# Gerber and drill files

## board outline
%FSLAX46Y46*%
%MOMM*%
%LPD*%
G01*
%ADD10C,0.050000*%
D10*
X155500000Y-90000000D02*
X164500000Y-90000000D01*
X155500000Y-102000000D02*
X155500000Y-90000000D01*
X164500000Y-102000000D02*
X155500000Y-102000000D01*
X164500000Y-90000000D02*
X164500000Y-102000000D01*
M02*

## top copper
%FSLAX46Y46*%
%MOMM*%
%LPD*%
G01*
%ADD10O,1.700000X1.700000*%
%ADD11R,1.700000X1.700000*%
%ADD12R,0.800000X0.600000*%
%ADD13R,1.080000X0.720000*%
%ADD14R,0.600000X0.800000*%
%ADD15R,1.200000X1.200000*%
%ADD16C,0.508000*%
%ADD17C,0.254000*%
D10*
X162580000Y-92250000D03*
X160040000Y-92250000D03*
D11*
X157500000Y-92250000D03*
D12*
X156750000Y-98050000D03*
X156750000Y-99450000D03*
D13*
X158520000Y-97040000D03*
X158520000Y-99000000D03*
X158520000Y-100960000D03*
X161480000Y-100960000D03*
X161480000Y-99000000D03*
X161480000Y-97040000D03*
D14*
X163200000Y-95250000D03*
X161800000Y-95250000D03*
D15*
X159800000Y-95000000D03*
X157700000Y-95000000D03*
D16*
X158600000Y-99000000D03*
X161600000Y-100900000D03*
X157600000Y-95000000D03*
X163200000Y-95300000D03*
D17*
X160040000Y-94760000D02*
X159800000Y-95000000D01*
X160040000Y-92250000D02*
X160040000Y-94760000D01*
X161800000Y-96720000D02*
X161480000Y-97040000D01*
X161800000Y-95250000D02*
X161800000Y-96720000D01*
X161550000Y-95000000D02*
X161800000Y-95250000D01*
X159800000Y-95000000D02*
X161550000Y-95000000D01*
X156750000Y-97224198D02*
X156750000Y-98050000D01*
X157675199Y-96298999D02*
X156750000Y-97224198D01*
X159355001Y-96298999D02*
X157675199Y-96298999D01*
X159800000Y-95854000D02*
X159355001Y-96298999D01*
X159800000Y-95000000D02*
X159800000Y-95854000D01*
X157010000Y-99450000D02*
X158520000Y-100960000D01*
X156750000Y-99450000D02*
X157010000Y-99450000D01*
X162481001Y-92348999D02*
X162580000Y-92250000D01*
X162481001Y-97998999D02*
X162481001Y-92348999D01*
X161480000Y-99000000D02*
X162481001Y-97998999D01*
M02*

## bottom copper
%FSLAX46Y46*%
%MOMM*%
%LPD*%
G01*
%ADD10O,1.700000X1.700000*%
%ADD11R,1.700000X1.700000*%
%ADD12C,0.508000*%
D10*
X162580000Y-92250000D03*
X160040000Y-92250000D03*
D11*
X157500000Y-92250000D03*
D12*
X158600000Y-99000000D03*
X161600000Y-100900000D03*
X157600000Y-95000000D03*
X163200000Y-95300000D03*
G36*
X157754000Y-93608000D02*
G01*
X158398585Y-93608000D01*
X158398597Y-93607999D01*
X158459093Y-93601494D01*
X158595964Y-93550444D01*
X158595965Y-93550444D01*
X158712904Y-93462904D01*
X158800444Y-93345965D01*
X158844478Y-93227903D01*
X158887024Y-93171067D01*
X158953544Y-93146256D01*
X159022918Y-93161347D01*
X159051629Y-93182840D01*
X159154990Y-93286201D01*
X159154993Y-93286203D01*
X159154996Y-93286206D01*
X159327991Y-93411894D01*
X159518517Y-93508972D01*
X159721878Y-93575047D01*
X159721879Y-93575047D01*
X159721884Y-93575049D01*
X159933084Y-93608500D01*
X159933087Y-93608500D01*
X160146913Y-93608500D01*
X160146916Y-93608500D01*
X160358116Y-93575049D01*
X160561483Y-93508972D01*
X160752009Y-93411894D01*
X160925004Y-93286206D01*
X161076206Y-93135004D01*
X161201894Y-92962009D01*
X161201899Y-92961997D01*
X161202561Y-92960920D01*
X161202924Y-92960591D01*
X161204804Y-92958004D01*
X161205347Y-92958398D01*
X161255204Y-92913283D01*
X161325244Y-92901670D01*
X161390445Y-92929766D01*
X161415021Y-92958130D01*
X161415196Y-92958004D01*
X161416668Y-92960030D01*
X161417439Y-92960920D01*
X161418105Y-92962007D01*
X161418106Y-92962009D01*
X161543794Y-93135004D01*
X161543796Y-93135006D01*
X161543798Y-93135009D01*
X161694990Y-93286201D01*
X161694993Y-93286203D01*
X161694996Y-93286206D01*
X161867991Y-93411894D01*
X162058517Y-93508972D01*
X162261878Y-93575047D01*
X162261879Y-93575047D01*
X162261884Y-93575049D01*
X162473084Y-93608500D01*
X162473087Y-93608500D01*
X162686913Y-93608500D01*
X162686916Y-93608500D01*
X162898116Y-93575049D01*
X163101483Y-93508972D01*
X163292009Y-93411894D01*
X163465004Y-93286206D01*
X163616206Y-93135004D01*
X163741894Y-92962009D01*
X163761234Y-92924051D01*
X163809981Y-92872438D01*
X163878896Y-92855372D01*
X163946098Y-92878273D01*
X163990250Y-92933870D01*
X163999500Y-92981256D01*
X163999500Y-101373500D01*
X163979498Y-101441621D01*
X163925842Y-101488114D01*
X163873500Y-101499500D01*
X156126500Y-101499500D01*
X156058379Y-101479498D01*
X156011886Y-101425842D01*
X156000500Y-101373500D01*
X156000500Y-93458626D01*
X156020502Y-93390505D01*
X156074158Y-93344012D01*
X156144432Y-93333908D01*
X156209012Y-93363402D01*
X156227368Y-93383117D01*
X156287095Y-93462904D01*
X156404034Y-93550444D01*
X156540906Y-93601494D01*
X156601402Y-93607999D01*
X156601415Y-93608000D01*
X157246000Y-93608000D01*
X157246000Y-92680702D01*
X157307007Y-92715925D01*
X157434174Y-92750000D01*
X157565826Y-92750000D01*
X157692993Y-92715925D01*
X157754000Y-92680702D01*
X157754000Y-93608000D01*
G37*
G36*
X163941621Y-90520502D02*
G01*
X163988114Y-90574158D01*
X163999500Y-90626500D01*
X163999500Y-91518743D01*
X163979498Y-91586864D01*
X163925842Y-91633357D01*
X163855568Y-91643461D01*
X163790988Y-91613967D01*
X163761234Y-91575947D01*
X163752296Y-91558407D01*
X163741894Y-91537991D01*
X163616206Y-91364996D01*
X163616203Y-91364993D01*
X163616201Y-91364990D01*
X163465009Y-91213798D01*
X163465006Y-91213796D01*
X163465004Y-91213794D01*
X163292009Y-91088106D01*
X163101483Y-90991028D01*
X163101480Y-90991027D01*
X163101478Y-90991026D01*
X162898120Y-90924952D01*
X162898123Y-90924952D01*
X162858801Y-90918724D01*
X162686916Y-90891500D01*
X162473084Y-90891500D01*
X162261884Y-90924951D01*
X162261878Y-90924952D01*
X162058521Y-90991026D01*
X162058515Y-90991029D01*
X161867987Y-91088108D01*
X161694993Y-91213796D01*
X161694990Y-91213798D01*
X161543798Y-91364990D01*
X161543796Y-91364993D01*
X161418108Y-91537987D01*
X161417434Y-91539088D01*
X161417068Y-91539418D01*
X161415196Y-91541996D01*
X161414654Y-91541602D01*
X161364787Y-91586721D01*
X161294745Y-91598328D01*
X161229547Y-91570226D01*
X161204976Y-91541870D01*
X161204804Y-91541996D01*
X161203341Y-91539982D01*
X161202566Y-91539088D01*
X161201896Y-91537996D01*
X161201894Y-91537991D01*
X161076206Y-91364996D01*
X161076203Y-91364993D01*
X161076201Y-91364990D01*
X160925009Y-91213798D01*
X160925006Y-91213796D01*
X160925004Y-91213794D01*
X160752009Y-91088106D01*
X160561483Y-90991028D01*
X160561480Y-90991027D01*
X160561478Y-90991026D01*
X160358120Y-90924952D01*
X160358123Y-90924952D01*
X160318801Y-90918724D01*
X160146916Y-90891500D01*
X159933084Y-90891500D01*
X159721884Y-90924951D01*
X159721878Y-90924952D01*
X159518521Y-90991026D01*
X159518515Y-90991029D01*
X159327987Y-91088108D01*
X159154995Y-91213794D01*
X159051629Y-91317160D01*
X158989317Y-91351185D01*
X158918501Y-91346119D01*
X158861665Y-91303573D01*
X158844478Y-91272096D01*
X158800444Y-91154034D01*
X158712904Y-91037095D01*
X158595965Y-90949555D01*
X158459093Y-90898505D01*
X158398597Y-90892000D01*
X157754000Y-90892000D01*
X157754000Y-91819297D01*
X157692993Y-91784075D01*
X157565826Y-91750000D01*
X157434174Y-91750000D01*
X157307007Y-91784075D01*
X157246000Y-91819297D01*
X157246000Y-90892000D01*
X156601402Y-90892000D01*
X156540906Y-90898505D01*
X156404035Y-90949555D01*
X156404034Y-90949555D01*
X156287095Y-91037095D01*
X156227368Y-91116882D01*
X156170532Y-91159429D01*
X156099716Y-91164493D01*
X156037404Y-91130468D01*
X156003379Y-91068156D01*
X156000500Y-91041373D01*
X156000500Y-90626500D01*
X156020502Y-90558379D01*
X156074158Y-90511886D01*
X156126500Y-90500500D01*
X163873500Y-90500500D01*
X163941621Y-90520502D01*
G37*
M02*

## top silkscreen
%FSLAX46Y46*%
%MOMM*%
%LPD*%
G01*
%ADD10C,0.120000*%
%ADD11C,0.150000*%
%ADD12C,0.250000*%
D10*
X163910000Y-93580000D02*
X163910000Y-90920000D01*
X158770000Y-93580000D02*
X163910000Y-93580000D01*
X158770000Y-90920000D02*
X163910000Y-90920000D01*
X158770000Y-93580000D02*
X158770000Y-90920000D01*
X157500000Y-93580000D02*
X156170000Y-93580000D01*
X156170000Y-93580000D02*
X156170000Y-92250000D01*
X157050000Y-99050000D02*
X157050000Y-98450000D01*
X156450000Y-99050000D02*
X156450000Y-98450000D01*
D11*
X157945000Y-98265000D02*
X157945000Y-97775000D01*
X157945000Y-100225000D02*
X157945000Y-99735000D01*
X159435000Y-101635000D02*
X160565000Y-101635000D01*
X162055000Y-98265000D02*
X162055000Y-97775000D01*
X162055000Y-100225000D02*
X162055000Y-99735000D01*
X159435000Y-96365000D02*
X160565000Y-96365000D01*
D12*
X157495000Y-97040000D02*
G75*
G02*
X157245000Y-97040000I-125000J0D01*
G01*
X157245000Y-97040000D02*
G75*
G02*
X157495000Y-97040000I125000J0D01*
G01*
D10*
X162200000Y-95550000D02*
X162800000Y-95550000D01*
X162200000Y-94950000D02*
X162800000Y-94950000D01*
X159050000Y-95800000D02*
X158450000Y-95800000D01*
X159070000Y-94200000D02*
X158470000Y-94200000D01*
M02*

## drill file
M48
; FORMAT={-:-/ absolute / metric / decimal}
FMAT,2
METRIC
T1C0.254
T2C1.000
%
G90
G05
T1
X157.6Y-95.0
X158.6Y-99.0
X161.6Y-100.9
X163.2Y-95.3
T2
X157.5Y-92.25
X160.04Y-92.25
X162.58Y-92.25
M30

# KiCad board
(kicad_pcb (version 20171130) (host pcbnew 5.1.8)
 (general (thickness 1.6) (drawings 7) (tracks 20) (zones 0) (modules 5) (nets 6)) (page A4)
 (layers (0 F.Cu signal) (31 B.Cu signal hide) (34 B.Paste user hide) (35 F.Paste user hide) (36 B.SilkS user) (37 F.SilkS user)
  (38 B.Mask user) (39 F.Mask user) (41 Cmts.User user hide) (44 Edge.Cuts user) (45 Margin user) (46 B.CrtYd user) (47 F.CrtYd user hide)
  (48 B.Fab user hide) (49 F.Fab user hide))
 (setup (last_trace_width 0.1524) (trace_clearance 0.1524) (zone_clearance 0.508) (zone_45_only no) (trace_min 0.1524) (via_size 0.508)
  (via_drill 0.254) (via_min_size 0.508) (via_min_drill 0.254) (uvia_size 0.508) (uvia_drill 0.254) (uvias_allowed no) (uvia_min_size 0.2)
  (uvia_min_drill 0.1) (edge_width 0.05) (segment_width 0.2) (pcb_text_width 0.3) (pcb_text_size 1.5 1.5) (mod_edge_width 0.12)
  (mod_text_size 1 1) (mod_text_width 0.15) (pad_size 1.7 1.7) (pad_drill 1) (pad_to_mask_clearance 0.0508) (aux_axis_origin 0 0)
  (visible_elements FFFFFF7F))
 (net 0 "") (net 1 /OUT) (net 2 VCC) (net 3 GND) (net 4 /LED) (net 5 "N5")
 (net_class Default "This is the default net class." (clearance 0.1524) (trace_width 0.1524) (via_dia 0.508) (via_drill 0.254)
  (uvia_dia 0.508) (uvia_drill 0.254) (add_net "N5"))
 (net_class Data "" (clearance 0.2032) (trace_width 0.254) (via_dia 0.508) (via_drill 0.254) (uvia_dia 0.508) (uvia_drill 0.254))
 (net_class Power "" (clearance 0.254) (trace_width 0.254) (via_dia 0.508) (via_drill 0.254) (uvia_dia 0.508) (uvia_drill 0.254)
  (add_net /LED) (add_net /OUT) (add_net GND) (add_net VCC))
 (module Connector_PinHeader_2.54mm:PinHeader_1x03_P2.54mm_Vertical (layer F.Cu) (at 157.5 92.25 90)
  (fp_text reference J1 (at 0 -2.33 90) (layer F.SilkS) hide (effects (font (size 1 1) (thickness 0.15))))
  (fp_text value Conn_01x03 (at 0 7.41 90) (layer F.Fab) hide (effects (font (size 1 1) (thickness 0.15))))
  (fp_line (start -1.33 6.41) (end 1.33 6.41) (layer F.SilkS) (width 0.12))
  (fp_line (start -1.33 1.27) (end -1.33 6.41) (layer F.SilkS) (width 0.12))
  (fp_line (start 1.33 1.27) (end 1.33 6.41) (layer F.SilkS) (width 0.12))
  (fp_line (start -1.33 1.27) (end 1.33 1.27) (layer F.SilkS) (width 0.12))
  (fp_line (start -1.33 0) (end -1.33 -1.33) (layer F.SilkS) (width 0.12))
  (fp_line (start -1.33 -1.33) (end 0 -1.33) (layer F.SilkS) (width 0.12))
  (pad 3 thru_hole oval (at 0 5.08 90) (size 1.7 1.7) (drill 1) (layers *.Cu *.Mask) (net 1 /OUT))
  (pad 2 thru_hole oval (at 0 2.54 90) (size 1.7 1.7) (drill 1) (layers *.Cu *.Mask) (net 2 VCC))
  (pad 1 thru_hole rect (at 0 0 90) (size 1.7 1.7) (drill 1) (layers *.Cu *.Mask) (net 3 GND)))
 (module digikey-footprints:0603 (layer F.Cu) (at 156.75 98.75 90)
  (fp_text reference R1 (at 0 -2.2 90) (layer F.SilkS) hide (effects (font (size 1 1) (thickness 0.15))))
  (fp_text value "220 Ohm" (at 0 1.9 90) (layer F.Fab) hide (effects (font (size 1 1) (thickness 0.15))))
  (fp_line (start -0.3 0.3) (end 0.3 0.3) (layer F.SilkS) (width 0.12))
  (fp_line (start -0.3 -0.3) (end 0.3 -0.3) (layer F.SilkS) (width 0.12))
  (pad 2 smd rect (at 0.7 0 90) (size 0.6 0.8) (layers F.Cu F.Paste F.Mask) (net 2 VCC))
  (pad 1 smd rect (at -0.7 0 90) (size 0.6 0.8) (layers F.Cu F.Paste F.Mask) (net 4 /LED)))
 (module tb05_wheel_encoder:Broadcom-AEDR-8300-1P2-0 (layer F.Cu) (at 160 99)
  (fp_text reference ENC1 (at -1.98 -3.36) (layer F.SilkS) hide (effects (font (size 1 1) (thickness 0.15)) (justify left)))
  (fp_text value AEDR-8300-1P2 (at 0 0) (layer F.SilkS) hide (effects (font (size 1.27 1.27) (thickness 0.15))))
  (fp_line (start -2.055 -0.735) (end -2.055 -1.225) (layer F.SilkS) (width 0.15))
  (fp_line (start -2.055 1.225) (end -2.055 0.735) (layer F.SilkS) (width 0.15))
  (fp_line (start -0.565 2.635) (end 0.565 2.635) (layer F.SilkS) (width 0.15))
  (fp_line (start 2.055 -0.735) (end 2.055 -1.225) (layer F.SilkS) (width 0.15))
  (fp_line (start 2.055 1.225) (end 2.055 0.735) (layer F.SilkS) (width 0.15))
  (fp_line (start -0.565 -2.635) (end 0.565 -2.635) (layer F.SilkS) (width 0.15))
  (fp_circle (center -2.63 -1.96) (end -2.505 -1.96) (layer F.SilkS) (width 0.25))
  (pad 1 smd rect (at -1.48 -1.96) (size 1.08 0.72) (layers F.Cu F.Paste F.Mask) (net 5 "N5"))
  (pad 2 smd rect (at -1.48 0) (size 1.08 0.72) (layers F.Cu F.Paste F.Mask) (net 3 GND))
  (pad 3 smd rect (at -1.48 1.96) (size 1.08 0.72) (layers F.Cu F.Paste F.Mask) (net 4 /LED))
  (pad 4 smd rect (at 1.48 1.96) (size 1.08 0.72) (layers F.Cu F.Paste F.Mask) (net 3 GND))
  (pad 5 smd rect (at 1.48 0) (size 1.08 0.72) (layers F.Cu F.Paste F.Mask) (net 1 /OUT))
  (pad 6 smd rect (at 1.48 -1.96) (size 1.08 0.72) (layers F.Cu F.Paste F.Mask) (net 2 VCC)))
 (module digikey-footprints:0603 (layer F.Cu) (at 162.5 95.25)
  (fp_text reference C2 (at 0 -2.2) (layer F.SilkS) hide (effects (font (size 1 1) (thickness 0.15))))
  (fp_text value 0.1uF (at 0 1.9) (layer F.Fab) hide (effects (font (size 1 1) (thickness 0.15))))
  (fp_line (start -0.3 0.3) (end 0.3 0.3) (layer F.SilkS) (width 0.12))
  (fp_line (start -0.3 -0.3) (end 0.3 -0.3) (layer F.SilkS) (width 0.12))
  (pad 2 smd rect (at 0.7 0) (size 0.6 0.8) (layers F.Cu F.Paste F.Mask) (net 3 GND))
  (pad 1 smd rect (at -0.7 0) (size 0.6 0.8) (layers F.Cu F.Paste F.Mask) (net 2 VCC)))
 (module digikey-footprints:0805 (layer F.Cu) (at 158.75 95 180)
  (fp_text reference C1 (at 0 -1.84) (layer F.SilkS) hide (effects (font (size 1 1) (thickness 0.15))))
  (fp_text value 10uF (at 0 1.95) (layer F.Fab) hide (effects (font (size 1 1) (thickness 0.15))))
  (fp_line (start -0.3 -0.8) (end 0.3 -0.8) (layer F.SilkS) (width 0.12))
  (fp_line (start -0.32 0.8) (end 0.28 0.8) (layer F.SilkS) (width 0.12))
  (pad 1 smd rect (at -1.05 0 180) (size 1.2 1.2) (layers F.Cu F.Paste F.Mask) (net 2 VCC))
  (pad 2 smd rect (at 1.05 0 180) (size 1.2 1.2) (layers F.Cu F.Paste F.Mask) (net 3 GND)))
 (gr_line (start 155.5 90) (end 164.5 90) (layer Edge.Cuts) (width 0.05))
 (gr_line (start 155.5 102) (end 155.5 90) (layer Edge.Cuts) (width 0.05))
 (gr_line (start 164.5 102) (end 155.5 102) (layer Edge.Cuts) (width 0.05))
 (gr_line (start 164.5 90) (end 164.5 102) (layer Edge.Cuts) (width 0.05))
 (via (at 158.6 99) (size 0.508) (drill 0.254) (layers F.Cu B.Cu) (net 3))
 (via (at 161.6 100.9) (size 0.508) (drill 0.254) (layers F.Cu B.Cu) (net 3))
 (via (at 157.6 95) (size 0.508) (drill 0.254) (layers F.Cu B.Cu) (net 3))
 (via (at 163.2 95.3) (size 0.508) (drill 0.254) (layers F.Cu B.Cu) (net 3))
 (segment (start 160.04 94.76) (end 159.8 95) (width 0.254) (layer F.Cu) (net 2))
 (segment (start 160.04 92.25) (end 160.04 94.76) (width 0.254) (layer F.Cu) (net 2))
 (segment (start 161.8 96.72) (end 161.48 97.04) (width 0.254) (layer F.Cu) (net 2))
 (segment (start 161.8 95.25) (end 161.8 96.72) (width 0.254) (layer F.Cu) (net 2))
 (segment (start 161.55 95) (end 161.8 95.25) (width 0.254) (layer F.Cu) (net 2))
 (segment (start 159.8 95) (end 161.55 95) (width 0.254) (layer F.Cu) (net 2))
 (segment (start 156.75 97.224198) (end 156.75 98.05) (width 0.254) (layer F.Cu) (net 2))
 (segment (start 157.675199 96.298999) (end 156.75 97.224198) (width 0.254) (layer F.Cu) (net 2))
 (segment (start 159.355001 96.298999) (end 157.675199 96.298999) (width 0.254) (layer F.Cu) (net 2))
 (segment (start 159.8 95.854) (end 159.355001 96.298999) (width 0.254) (layer F.Cu) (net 2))
 (segment (start 159.8 95) (end 159.8 95.854) (width 0.254) (layer F.Cu) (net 2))
 (segment (start 157.01 99.45) (end 158.52 100.96) (width 0.254) (layer F.Cu) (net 4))
 (segment (start 156.75 99.45) (end 157.01 99.45) (width 0.254) (layer F.Cu) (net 4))
 (segment (start 162.481001 92.348999) (end 162.58 92.25) (width 0.254) (layer F.Cu) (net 1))
 (segment (start 162.481001 97.998999) (end 162.481001 92.348999) (width 0.254) (layer F.Cu) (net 1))
 (segment (start 161.48 99) (end 162.481001 97.998999) (width 0.254) (layer F.Cu) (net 1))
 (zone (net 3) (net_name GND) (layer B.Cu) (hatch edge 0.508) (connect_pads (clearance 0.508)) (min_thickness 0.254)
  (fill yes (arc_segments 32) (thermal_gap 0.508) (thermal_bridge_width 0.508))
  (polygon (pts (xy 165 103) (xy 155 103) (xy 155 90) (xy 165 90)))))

